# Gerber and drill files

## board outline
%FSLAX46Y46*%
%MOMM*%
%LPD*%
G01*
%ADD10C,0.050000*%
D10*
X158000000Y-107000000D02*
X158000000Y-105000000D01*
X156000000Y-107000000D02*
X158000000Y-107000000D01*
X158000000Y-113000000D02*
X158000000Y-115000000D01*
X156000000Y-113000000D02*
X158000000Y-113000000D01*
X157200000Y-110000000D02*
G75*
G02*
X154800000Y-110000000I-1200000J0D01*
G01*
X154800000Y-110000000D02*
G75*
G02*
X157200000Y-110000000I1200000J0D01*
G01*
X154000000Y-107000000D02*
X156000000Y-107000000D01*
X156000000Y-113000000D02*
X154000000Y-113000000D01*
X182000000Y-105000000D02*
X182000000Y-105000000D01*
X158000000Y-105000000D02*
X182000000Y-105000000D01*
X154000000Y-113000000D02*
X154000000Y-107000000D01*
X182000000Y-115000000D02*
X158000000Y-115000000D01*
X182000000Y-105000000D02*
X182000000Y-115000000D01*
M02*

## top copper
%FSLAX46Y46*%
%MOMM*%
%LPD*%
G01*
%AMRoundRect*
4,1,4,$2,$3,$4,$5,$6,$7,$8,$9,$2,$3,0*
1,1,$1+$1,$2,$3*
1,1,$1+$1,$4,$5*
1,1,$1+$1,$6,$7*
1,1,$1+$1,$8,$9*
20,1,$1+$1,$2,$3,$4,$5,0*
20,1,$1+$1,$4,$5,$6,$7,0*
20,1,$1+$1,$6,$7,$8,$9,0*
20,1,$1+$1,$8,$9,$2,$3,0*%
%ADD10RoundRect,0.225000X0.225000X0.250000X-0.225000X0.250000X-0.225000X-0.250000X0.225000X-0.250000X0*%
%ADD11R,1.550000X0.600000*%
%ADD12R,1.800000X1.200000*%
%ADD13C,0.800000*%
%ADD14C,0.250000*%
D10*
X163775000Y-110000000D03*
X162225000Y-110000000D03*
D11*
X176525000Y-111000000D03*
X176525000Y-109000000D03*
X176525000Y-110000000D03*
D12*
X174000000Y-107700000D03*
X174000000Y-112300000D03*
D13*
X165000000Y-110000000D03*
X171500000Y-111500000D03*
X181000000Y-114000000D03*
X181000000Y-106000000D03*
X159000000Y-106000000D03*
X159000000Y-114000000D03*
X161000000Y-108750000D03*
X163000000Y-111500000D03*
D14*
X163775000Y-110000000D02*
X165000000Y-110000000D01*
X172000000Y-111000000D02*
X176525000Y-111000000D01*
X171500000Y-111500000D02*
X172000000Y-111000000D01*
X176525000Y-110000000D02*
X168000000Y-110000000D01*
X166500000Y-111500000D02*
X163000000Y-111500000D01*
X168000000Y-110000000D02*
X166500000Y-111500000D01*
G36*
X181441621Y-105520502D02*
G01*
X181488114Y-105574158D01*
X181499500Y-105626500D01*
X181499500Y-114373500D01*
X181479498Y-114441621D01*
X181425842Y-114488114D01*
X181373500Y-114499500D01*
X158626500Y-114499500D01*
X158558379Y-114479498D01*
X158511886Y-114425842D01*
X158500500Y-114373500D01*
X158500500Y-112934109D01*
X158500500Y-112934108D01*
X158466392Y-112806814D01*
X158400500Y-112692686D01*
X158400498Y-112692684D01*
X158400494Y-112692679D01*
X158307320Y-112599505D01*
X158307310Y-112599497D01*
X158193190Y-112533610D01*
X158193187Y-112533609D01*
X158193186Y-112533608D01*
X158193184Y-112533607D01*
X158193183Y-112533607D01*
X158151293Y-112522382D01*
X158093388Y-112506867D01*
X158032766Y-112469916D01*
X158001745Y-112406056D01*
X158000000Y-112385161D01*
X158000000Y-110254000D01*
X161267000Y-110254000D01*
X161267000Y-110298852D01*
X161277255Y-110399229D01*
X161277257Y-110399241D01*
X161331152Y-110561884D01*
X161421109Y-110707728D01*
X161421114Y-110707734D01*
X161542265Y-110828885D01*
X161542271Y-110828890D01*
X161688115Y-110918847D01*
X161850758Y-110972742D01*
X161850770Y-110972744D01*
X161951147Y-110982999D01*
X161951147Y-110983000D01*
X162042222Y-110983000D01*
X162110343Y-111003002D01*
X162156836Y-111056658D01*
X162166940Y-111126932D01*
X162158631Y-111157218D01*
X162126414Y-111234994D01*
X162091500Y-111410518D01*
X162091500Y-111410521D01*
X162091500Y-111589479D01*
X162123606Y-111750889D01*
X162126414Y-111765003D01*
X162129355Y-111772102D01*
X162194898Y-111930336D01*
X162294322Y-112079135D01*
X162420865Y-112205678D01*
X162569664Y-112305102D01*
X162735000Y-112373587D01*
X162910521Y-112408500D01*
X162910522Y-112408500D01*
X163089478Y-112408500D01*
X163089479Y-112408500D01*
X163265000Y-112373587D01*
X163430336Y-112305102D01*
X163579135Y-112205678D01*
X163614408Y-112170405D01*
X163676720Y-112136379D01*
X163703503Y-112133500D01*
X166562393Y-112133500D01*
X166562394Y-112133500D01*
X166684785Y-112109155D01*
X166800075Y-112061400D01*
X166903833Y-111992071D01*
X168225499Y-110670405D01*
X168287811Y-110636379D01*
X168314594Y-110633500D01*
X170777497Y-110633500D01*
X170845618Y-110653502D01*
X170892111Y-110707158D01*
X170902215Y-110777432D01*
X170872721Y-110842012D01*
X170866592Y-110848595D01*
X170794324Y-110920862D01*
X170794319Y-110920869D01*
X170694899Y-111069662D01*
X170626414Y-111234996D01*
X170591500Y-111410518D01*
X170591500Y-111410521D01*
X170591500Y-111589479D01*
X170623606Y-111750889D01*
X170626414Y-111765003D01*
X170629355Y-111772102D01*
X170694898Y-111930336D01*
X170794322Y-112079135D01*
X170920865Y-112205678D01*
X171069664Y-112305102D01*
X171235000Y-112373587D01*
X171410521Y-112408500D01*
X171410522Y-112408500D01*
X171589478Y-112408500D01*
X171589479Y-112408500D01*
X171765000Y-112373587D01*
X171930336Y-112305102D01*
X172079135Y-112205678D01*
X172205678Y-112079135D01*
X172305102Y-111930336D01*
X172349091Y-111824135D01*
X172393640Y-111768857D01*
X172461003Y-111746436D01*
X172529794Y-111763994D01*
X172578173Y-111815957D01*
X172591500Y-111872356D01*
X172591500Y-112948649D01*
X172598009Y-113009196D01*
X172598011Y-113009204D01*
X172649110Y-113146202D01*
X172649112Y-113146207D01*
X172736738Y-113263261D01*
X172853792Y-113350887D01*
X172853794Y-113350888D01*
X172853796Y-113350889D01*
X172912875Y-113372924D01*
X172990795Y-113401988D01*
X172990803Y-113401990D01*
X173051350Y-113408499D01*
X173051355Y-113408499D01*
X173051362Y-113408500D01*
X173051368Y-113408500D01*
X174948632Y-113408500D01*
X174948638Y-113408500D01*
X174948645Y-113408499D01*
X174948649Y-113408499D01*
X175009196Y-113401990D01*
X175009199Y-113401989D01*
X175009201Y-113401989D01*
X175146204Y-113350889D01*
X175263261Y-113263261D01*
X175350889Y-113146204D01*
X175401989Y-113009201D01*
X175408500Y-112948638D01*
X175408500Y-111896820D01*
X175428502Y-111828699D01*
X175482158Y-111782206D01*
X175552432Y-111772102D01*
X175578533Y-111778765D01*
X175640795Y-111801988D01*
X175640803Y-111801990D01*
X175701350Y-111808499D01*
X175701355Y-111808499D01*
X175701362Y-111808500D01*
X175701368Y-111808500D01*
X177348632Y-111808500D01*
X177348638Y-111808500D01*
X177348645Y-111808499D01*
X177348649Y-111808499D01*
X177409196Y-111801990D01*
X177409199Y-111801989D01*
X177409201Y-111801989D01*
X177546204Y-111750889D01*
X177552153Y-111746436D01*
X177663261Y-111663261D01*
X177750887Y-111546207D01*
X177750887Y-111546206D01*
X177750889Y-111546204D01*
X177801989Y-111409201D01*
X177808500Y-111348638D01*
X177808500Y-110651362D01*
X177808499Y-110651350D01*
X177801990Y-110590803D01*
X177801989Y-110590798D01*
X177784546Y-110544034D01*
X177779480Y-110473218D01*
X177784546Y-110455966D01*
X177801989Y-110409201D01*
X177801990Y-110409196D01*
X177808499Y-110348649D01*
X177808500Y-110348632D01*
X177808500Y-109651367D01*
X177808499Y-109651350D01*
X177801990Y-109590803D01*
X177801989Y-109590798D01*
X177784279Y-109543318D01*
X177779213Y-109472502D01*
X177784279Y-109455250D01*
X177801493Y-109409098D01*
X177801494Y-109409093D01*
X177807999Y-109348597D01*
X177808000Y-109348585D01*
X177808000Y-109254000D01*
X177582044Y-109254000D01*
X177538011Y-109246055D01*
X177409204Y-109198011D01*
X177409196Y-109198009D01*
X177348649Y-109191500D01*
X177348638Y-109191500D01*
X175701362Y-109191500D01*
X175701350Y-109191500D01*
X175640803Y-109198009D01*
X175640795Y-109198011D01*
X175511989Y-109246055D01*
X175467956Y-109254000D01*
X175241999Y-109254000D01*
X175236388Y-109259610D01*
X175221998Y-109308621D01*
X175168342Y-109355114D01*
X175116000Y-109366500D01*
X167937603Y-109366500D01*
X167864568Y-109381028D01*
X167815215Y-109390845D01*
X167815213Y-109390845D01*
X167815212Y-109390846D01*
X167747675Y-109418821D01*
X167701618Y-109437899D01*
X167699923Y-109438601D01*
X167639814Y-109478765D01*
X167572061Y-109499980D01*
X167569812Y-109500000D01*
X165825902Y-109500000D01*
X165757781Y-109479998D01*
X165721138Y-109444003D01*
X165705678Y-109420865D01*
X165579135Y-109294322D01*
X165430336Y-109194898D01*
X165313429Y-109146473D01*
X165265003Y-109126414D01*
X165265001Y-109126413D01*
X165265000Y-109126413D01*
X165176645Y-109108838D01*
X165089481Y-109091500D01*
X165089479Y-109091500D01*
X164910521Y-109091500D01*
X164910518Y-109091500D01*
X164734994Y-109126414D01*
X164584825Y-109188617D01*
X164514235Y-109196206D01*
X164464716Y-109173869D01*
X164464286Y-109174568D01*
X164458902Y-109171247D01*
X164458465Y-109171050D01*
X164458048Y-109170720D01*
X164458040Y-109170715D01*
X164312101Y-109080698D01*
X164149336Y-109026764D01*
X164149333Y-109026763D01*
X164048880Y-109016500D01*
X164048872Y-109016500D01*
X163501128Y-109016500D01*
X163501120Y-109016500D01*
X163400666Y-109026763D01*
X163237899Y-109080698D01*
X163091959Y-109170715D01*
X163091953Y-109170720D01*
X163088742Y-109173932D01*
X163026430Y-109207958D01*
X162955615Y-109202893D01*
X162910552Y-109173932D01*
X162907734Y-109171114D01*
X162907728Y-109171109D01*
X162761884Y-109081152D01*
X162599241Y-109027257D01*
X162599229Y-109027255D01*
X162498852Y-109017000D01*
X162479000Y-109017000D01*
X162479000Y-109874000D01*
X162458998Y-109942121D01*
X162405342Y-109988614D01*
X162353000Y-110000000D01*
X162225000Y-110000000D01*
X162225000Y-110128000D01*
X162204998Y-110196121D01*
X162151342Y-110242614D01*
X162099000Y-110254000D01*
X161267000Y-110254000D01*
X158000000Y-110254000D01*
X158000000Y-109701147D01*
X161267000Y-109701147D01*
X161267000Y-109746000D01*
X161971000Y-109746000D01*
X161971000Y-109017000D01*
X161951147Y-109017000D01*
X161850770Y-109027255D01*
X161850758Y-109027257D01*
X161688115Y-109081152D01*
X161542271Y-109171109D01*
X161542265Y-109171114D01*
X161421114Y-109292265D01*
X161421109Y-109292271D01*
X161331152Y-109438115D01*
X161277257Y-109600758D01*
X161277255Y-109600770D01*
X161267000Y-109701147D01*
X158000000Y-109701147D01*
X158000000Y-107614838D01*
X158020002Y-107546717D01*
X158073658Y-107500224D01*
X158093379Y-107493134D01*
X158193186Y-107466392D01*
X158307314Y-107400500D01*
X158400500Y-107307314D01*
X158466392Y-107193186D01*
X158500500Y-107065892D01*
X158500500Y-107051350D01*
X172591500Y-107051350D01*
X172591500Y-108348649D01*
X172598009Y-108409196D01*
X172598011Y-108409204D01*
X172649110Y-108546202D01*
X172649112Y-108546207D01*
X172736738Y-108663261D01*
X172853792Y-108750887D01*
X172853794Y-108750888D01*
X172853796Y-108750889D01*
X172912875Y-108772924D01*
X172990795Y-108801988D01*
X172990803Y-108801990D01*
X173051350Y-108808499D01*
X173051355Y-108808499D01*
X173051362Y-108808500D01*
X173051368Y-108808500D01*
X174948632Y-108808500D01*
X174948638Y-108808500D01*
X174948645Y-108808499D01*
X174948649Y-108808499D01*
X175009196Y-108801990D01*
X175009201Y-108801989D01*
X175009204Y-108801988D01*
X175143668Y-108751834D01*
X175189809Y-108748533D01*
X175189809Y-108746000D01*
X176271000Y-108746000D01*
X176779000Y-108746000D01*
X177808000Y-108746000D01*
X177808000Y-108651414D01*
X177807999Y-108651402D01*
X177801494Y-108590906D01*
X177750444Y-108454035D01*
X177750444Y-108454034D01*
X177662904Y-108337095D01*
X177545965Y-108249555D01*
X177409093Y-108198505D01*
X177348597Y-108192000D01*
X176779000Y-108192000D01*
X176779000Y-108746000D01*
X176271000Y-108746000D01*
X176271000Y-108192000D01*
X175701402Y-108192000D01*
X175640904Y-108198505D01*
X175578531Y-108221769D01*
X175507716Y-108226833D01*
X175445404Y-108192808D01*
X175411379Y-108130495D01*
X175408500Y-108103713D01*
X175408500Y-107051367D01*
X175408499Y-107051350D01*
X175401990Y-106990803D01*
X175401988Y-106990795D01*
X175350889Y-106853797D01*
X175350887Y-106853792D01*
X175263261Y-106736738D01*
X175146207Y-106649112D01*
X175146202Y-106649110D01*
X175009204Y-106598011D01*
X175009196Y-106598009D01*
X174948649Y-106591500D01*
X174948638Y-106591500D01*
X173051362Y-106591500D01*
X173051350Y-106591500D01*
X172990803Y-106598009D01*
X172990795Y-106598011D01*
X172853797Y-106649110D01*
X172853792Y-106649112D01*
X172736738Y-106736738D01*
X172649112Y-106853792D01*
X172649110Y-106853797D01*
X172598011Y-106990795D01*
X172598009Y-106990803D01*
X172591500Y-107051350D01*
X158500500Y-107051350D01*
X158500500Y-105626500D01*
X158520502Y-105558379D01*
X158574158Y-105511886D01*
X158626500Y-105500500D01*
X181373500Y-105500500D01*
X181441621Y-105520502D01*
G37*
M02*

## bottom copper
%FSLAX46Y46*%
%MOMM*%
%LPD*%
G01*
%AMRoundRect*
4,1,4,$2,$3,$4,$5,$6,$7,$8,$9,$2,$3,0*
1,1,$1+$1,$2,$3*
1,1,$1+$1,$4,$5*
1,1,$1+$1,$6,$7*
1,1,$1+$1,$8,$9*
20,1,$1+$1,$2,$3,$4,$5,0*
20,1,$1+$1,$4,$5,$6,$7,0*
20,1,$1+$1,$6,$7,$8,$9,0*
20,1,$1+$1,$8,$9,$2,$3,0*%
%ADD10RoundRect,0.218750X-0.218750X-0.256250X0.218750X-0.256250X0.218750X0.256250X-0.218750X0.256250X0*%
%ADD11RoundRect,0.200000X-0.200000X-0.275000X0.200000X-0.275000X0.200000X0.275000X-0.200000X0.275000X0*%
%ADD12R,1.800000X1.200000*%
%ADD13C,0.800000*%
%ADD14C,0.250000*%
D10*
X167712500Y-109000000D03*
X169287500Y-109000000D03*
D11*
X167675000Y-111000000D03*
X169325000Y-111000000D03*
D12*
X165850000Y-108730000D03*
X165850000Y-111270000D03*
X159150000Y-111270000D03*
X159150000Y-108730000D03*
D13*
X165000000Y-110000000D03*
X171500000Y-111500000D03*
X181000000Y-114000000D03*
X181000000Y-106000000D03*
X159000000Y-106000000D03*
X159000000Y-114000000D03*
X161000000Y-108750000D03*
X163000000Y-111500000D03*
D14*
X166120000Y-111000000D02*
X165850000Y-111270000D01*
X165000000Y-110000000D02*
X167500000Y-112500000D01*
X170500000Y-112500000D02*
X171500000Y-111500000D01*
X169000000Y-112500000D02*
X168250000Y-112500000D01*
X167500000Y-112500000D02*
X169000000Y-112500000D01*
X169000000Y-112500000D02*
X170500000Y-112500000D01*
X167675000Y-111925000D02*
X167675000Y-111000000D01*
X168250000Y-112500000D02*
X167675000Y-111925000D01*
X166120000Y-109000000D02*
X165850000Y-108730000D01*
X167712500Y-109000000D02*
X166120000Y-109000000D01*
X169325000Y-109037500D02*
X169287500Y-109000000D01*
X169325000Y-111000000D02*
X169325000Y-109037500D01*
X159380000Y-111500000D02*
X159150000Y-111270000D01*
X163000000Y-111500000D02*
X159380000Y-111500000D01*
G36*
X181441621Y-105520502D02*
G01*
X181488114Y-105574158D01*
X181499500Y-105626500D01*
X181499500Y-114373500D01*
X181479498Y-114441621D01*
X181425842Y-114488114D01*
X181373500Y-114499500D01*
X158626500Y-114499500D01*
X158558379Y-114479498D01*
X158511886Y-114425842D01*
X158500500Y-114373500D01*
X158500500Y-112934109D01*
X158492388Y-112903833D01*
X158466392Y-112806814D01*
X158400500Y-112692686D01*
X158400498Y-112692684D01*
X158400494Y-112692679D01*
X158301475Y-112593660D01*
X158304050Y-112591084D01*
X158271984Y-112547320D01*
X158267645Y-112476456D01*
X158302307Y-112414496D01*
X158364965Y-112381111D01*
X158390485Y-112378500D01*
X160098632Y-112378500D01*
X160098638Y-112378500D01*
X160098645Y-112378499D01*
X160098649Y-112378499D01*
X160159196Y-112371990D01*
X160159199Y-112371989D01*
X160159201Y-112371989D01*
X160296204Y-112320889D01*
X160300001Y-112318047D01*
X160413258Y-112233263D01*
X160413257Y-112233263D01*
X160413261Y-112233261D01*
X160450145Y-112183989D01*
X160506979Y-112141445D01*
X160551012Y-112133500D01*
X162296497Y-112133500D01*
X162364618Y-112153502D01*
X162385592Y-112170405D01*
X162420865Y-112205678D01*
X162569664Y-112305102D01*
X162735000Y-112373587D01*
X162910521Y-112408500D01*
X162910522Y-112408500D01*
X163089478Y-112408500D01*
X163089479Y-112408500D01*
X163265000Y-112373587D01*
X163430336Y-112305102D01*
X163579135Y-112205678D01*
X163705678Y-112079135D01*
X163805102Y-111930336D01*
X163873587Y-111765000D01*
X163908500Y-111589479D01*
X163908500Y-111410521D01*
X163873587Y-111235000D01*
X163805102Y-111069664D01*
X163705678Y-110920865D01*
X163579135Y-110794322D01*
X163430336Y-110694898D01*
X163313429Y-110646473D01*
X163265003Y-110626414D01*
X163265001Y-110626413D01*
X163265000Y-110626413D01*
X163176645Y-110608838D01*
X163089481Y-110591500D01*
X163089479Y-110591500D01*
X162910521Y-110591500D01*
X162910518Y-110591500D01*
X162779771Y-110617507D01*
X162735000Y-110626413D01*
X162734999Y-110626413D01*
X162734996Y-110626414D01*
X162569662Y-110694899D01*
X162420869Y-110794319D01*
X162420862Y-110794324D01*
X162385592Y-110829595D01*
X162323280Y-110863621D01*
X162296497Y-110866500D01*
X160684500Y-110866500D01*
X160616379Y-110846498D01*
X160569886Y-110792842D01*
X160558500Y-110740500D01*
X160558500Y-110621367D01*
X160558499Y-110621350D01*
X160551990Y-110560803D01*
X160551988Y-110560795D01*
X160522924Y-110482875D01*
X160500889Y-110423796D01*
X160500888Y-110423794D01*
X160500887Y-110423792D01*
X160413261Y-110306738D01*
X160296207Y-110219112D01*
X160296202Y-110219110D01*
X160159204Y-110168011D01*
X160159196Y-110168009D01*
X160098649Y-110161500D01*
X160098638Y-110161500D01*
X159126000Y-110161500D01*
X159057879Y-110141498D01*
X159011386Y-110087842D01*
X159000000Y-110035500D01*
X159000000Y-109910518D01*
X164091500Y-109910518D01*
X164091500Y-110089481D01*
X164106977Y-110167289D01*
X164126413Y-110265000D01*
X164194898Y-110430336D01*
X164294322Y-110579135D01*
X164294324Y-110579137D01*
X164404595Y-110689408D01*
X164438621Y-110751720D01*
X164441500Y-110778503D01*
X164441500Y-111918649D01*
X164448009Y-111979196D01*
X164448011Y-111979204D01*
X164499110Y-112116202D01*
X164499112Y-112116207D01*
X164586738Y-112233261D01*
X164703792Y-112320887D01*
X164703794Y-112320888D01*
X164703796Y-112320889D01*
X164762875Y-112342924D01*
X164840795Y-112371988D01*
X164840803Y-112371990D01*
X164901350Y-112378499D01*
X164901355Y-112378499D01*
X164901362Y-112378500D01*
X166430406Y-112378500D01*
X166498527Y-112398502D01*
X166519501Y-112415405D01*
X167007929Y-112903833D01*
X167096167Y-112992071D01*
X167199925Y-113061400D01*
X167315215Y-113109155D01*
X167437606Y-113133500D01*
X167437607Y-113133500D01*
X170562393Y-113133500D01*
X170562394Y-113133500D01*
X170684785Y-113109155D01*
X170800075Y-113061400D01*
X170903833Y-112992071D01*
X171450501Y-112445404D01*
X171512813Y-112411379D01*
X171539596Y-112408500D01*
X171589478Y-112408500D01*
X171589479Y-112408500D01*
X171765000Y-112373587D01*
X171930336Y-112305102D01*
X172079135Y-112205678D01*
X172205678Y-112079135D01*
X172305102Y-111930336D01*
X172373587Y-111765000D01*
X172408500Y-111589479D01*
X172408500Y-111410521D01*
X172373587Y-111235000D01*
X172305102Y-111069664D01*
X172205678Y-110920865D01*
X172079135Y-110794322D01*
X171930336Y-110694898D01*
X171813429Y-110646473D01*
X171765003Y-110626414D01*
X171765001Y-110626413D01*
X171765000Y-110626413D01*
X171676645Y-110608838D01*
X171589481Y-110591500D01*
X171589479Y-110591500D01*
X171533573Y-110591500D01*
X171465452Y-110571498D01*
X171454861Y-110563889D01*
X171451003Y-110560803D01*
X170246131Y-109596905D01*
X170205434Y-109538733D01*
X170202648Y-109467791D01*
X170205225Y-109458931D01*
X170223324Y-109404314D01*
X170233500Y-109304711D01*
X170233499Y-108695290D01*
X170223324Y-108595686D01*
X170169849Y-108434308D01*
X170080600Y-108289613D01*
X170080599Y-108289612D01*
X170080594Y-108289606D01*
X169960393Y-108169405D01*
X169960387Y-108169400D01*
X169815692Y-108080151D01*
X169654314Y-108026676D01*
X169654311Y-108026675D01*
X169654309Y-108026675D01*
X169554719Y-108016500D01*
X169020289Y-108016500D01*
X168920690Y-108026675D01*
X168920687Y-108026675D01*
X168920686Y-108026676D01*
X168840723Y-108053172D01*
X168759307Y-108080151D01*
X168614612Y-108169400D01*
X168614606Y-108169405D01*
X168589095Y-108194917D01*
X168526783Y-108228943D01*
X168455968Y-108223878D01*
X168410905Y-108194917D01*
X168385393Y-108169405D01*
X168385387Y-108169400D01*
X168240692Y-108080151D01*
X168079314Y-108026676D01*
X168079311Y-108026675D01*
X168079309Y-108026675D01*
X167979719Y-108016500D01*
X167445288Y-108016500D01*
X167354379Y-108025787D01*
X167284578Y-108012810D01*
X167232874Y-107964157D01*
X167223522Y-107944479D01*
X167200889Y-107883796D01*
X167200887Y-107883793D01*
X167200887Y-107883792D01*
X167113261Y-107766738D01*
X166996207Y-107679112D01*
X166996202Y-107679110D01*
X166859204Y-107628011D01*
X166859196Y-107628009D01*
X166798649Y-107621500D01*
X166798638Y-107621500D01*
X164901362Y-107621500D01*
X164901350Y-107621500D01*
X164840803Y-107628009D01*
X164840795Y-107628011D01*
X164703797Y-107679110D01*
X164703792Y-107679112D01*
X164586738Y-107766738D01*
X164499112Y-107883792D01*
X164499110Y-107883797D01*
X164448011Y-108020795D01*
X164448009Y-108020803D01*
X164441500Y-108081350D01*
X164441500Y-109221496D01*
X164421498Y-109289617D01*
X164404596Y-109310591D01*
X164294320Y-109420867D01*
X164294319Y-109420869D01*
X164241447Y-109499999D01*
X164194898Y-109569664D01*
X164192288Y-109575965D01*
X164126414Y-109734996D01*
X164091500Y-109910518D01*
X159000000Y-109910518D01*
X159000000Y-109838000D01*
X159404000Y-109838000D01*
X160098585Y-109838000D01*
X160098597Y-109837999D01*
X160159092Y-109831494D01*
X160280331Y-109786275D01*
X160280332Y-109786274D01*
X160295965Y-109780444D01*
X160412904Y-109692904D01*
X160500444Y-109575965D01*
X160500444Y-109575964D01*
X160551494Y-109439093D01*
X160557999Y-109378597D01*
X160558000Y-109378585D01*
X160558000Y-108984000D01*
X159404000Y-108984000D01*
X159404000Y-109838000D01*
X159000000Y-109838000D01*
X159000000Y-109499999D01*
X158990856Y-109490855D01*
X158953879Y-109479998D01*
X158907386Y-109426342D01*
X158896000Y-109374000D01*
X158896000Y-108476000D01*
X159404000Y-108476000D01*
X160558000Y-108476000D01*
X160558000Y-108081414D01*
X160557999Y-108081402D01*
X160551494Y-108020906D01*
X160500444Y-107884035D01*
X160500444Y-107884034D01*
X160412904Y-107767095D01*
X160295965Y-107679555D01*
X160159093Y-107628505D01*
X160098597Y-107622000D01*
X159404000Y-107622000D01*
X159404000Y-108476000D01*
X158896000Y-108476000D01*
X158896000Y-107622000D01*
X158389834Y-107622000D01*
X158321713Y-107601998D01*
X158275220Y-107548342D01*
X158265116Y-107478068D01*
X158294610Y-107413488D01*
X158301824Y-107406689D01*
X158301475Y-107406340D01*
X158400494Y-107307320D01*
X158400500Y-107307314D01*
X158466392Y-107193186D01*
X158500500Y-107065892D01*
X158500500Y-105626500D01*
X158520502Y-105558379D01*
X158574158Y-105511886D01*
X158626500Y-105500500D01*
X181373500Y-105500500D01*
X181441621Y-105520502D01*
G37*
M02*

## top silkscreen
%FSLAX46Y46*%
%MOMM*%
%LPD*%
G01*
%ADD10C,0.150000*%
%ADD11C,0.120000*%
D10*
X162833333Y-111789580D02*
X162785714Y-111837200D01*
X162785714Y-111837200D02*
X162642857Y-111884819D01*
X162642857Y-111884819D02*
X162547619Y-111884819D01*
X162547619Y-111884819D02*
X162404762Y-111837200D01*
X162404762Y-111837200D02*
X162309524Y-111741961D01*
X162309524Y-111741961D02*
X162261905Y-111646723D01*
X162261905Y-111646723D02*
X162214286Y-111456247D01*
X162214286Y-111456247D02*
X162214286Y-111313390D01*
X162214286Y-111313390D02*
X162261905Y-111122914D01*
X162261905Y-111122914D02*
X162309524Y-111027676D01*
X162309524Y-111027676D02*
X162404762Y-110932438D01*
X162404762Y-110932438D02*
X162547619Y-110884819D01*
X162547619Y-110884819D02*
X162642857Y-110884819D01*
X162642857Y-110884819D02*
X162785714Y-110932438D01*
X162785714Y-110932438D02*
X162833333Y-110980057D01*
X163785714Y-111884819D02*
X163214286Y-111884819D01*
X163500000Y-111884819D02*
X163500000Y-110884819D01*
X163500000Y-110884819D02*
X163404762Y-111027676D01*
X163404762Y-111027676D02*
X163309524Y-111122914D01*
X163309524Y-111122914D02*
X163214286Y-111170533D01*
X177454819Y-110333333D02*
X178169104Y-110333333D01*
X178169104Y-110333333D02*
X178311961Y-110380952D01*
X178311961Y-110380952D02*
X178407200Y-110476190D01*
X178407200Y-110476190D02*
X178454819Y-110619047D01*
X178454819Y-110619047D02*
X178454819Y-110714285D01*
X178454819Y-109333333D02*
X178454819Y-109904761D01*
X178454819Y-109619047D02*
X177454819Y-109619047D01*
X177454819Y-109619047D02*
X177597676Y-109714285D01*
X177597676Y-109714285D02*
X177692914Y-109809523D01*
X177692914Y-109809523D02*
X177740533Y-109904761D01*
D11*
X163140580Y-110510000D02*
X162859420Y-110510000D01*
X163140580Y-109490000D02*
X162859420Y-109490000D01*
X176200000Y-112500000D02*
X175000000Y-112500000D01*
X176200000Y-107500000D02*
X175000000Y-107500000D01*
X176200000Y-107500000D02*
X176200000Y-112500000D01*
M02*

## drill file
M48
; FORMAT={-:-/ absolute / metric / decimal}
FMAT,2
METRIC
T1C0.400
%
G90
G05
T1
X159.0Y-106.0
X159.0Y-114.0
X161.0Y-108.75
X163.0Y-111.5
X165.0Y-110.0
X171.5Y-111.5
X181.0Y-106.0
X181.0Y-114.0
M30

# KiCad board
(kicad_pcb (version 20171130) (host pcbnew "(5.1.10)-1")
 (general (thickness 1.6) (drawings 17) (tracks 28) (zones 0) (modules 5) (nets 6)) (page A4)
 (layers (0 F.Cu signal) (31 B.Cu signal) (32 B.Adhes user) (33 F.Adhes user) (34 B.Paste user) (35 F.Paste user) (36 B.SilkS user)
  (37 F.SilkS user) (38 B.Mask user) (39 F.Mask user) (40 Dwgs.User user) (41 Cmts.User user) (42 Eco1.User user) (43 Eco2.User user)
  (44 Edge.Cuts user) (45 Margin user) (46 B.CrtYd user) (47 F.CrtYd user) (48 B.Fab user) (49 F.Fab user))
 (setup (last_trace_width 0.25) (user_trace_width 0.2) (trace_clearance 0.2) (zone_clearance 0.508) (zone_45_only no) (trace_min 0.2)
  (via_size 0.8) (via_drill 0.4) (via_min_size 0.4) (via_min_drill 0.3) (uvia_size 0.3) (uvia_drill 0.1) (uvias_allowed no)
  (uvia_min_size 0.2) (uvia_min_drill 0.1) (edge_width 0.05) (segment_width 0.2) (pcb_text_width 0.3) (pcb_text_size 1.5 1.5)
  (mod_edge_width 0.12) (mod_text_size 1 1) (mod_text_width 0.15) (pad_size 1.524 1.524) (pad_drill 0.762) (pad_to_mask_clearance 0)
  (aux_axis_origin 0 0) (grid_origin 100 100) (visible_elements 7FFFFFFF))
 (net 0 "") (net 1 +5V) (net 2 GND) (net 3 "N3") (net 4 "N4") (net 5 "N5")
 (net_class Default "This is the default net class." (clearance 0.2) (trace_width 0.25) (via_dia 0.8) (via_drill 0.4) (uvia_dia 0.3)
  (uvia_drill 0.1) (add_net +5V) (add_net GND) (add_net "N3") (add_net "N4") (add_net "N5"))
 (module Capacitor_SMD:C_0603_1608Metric (layer F.Cu) (at 163 110 180)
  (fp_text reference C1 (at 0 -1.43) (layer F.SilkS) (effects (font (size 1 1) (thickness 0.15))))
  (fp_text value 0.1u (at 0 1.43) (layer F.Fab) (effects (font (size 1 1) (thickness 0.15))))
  (fp_line (start -0.14058 -0.51) (end 0.14058 -0.51) (layer F.SilkS) (width 0.12))
  (fp_line (start -0.14058 0.51) (end 0.14058 0.51) (layer F.SilkS) (width 0.12))
  (pad 1 smd roundrect (at -0.775 0 180) (size 0.9 0.95) (layers F.Cu F.Paste F.Mask) (roundrect_rratio 0.25) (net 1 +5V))
  (pad 2 smd roundrect (at 0.775 0 180) (size 0.9 0.95) (layers F.Cu F.Paste F.Mask) (roundrect_rratio 0.25) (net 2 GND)))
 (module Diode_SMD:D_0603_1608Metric (layer B.Cu) (at 168.5 109)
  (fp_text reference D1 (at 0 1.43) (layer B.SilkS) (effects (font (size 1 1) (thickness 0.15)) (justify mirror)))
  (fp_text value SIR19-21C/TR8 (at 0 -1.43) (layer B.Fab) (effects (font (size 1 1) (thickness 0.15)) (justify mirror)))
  (pad 1 smd roundrect (at -0.7875 0) (size 0.875 0.95) (layers B.Cu B.Paste B.Mask) (roundrect_rratio 0.25) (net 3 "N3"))
  (pad 2 smd roundrect (at 0.7875 0) (size 0.875 0.95) (layers B.Cu B.Paste B.Mask) (roundrect_rratio 0.25) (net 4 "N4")))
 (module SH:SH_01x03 (layer F.Cu) (at 174 110 270)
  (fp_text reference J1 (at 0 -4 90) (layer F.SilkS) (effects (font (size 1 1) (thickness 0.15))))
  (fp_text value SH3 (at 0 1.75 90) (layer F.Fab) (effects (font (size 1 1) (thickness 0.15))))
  (fp_line (start 2.5 -2.2) (end 2.5 -1) (layer F.SilkS) (width 0.12))
  (fp_line (start -2.5 -2.2) (end -2.5 -1) (layer F.SilkS) (width 0.12))
  (fp_line (start -2.5 -2.2) (end 2.5 -2.2) (layer F.SilkS) (width 0.12))
  (pad 3 smd rect (at 1 -2.525 270) (size 0.6 1.55) (layers F.Cu F.Paste F.Mask) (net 1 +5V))
  (pad 1 smd rect (at -1 -2.525 270) (size 0.6 1.55) (layers F.Cu F.Paste F.Mask) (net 2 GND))
  (pad 2 smd rect (at 0 -2.525 270) (size 0.6 1.55) (layers F.Cu F.Paste F.Mask) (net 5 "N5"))
  (pad MP smd rect (at -2.3 0 270) (size 1.2 1.8) (layers F.Cu F.Paste F.Mask))
  (pad MP smd rect (at 2.3 0 270) (size 1.2 1.8) (layers F.Cu F.Paste F.Mask)))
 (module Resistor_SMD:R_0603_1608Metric (layer B.Cu) (at 168.5 111)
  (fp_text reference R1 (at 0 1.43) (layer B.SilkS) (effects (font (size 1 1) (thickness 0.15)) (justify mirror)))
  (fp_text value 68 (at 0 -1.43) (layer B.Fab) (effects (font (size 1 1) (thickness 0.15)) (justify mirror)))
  (pad 1 smd roundrect (at -0.825 0) (size 0.8 0.95) (layers B.Cu B.Paste B.Mask) (roundrect_rratio 0.25) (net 1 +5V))
  (pad 2 smd roundrect (at 0.825 0) (size 0.8 0.95) (layers B.Cu B.Paste B.Mask) (roundrect_rratio 0.25) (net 4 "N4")))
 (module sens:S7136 (layer B.Cu) (at 162.5 110 180)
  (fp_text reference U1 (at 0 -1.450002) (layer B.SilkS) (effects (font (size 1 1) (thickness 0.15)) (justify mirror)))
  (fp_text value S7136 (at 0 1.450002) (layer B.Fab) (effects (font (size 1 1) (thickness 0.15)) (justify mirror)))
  (pad 1 smd rect (at -3.35 1.27 180) (size 1.8 1.2) (layers B.Cu B.Paste B.Mask) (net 3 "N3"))
  (pad 2 smd rect (at -3.35 -1.27 180) (size 1.8 1.2) (layers B.Cu B.Paste B.Mask) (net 1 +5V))
  (pad 3 smd rect (at 3.35 -1.27 180) (size 1.8 1.2) (layers B.Cu B.Paste B.Mask) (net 5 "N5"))
  (pad 4 smd rect (at 3.35 1.27 180) (size 1.8 1.2) (layers B.Cu B.Paste B.Mask) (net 2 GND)))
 (gr_line (start 158 107) (end 158 105) (layer Edge.Cuts) (width 0.05))
 (gr_line (start 156 107) (end 158 107) (layer Edge.Cuts) (width 0.05))
 (gr_line (start 158 113) (end 158 115) (layer Edge.Cuts) (width 0.05))
 (gr_line (start 156 113) (end 158 113) (layer Edge.Cuts) (width 0.05))
 (gr_circle (center 156 110) (end 157.2 110) (layer Edge.Cuts) (width 0.05))
 (gr_line (start 154 107) (end 156 107) (layer Edge.Cuts) (width 0.05))
 (gr_line (start 156 113) (end 154 113) (layer Edge.Cuts) (width 0.05))
 (gr_line (start 182 105) (end 182 105) (layer Edge.Cuts) (width 0.05))
 (gr_line (start 158 105) (end 182 105) (layer Edge.Cuts) (width 0.05))
 (gr_line (start 154 113) (end 154 107) (layer Edge.Cuts) (width 0.05))
 (gr_line (start 182 115) (end 158 115) (layer Edge.Cuts) (width 0.05))
 (gr_line (start 182 105) (end 182 115) (layer Edge.Cuts) (width 0.05))
 (segment (start 166.12 111) (end 165.85 111.27) (width 0.25) (layer B.Cu) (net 1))
 (via (at 165 110) (size 0.8) (drill 0.4) (layers F.Cu B.Cu) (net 1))
 (segment (start 163.775 110) (end 165 110) (width 0.25) (layer F.Cu) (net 1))
 (segment (start 165 110) (end 167.5 112.5) (width 0.25) (layer B.Cu) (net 1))
 (via (at 171.5 111.5) (size 0.8) (drill 0.4) (layers F.Cu B.Cu) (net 1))
 (segment (start 170.5 112.5) (end 171.5 111.5) (width 0.25) (layer B.Cu) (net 1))
 (segment (start 172 111) (end 176.525 111) (width 0.25) (layer F.Cu) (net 1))
 (segment (start 171.5 111.5) (end 172 111) (width 0.25) (layer F.Cu) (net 1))
 (segment (start 169 112.5) (end 168.25 112.5) (width 0.25) (layer B.Cu) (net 1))
 (segment (start 167.5 112.5) (end 169 112.5) (width 0.25) (layer B.Cu) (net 1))
 (segment (start 169 112.5) (end 170.5 112.5) (width 0.25) (layer B.Cu) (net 1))
 (segment (start 167.675 111.925) (end 167.675 111) (width 0.25) (layer B.Cu) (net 1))
 (segment (start 168.25 112.5) (end 167.675 111.925) (width 0.25) (layer B.Cu) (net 1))
 (via (at 181 114) (size 0.8) (drill 0.4) (layers F.Cu B.Cu) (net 2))
 (via (at 181 106) (size 0.8) (drill 0.4) (layers F.Cu B.Cu) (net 2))
 (via (at 159 106) (size 0.8) (drill 0.4) (layers F.Cu B.Cu) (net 2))
 (via (at 159 114) (size 0.8) (drill 0.4) (layers F.Cu B.Cu) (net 2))
 (via (at 161 108.75) (size 0.8) (drill 0.4) (layers F.Cu B.Cu) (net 2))
 (segment (start 166.12 109) (end 165.85 108.73) (width 0.25) (layer B.Cu) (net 3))
 (segment (start 167.7125 109) (end 166.12 109) (width 0.25) (layer B.Cu) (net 3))
 (segment (start 169.325 109.0375) (end 169.2875 109) (width 0.25) (layer B.Cu) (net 4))
 (segment (start 169.325 111) (end 169.325 109.0375) (width 0.25) (layer B.Cu) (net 4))
 (segment (start 176.525 110) (end 168 110) (width 0.25) (layer F.Cu) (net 5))
 (via (at 163 111.5) (size 0.8) (drill 0.4) (layers F.Cu B.Cu) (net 5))
 (segment (start 166.5 111.5) (end 163 111.5) (width 0.25) (layer F.Cu) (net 5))
 (segment (start 168 110) (end 166.5 111.5) (width 0.25) (layer F.Cu) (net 5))
 (segment (start 159.38 111.5) (end 159.15 111.27) (width 0.25) (layer B.Cu) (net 5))
 (segment (start 163 111.5) (end 159.38 111.5) (width 0.25) (layer B.Cu) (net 5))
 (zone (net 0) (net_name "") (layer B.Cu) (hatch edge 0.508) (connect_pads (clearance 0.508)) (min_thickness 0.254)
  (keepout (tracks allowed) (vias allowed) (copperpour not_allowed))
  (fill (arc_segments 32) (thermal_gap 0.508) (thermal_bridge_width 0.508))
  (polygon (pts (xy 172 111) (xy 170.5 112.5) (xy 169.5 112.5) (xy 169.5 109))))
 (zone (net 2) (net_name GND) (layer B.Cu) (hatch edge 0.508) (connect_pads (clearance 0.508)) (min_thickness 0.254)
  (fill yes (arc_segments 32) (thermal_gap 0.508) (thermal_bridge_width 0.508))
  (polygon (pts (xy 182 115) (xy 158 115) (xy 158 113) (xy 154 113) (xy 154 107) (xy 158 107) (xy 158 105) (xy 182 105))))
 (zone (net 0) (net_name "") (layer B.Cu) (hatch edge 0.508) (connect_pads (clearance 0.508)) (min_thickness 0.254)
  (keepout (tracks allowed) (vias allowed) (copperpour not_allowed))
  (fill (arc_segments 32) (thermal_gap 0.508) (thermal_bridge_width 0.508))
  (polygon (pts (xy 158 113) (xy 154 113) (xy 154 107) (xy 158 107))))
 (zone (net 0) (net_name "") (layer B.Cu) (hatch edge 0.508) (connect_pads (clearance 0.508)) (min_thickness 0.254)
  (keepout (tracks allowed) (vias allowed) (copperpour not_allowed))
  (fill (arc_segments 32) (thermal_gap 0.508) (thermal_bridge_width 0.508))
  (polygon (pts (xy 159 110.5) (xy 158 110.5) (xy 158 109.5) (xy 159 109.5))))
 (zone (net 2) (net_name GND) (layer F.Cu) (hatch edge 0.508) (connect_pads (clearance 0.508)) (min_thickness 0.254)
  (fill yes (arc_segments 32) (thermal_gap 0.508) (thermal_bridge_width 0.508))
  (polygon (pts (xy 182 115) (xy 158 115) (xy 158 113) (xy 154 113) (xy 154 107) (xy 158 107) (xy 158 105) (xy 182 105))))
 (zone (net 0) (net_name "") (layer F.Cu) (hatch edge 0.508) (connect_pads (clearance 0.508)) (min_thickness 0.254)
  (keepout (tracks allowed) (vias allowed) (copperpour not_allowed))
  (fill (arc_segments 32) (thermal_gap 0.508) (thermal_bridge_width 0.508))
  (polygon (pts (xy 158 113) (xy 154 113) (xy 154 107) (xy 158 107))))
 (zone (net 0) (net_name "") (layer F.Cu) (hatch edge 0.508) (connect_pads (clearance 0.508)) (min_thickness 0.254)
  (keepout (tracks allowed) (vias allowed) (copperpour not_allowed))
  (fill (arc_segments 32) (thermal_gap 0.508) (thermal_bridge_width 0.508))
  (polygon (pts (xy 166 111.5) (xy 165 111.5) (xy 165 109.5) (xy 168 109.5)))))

